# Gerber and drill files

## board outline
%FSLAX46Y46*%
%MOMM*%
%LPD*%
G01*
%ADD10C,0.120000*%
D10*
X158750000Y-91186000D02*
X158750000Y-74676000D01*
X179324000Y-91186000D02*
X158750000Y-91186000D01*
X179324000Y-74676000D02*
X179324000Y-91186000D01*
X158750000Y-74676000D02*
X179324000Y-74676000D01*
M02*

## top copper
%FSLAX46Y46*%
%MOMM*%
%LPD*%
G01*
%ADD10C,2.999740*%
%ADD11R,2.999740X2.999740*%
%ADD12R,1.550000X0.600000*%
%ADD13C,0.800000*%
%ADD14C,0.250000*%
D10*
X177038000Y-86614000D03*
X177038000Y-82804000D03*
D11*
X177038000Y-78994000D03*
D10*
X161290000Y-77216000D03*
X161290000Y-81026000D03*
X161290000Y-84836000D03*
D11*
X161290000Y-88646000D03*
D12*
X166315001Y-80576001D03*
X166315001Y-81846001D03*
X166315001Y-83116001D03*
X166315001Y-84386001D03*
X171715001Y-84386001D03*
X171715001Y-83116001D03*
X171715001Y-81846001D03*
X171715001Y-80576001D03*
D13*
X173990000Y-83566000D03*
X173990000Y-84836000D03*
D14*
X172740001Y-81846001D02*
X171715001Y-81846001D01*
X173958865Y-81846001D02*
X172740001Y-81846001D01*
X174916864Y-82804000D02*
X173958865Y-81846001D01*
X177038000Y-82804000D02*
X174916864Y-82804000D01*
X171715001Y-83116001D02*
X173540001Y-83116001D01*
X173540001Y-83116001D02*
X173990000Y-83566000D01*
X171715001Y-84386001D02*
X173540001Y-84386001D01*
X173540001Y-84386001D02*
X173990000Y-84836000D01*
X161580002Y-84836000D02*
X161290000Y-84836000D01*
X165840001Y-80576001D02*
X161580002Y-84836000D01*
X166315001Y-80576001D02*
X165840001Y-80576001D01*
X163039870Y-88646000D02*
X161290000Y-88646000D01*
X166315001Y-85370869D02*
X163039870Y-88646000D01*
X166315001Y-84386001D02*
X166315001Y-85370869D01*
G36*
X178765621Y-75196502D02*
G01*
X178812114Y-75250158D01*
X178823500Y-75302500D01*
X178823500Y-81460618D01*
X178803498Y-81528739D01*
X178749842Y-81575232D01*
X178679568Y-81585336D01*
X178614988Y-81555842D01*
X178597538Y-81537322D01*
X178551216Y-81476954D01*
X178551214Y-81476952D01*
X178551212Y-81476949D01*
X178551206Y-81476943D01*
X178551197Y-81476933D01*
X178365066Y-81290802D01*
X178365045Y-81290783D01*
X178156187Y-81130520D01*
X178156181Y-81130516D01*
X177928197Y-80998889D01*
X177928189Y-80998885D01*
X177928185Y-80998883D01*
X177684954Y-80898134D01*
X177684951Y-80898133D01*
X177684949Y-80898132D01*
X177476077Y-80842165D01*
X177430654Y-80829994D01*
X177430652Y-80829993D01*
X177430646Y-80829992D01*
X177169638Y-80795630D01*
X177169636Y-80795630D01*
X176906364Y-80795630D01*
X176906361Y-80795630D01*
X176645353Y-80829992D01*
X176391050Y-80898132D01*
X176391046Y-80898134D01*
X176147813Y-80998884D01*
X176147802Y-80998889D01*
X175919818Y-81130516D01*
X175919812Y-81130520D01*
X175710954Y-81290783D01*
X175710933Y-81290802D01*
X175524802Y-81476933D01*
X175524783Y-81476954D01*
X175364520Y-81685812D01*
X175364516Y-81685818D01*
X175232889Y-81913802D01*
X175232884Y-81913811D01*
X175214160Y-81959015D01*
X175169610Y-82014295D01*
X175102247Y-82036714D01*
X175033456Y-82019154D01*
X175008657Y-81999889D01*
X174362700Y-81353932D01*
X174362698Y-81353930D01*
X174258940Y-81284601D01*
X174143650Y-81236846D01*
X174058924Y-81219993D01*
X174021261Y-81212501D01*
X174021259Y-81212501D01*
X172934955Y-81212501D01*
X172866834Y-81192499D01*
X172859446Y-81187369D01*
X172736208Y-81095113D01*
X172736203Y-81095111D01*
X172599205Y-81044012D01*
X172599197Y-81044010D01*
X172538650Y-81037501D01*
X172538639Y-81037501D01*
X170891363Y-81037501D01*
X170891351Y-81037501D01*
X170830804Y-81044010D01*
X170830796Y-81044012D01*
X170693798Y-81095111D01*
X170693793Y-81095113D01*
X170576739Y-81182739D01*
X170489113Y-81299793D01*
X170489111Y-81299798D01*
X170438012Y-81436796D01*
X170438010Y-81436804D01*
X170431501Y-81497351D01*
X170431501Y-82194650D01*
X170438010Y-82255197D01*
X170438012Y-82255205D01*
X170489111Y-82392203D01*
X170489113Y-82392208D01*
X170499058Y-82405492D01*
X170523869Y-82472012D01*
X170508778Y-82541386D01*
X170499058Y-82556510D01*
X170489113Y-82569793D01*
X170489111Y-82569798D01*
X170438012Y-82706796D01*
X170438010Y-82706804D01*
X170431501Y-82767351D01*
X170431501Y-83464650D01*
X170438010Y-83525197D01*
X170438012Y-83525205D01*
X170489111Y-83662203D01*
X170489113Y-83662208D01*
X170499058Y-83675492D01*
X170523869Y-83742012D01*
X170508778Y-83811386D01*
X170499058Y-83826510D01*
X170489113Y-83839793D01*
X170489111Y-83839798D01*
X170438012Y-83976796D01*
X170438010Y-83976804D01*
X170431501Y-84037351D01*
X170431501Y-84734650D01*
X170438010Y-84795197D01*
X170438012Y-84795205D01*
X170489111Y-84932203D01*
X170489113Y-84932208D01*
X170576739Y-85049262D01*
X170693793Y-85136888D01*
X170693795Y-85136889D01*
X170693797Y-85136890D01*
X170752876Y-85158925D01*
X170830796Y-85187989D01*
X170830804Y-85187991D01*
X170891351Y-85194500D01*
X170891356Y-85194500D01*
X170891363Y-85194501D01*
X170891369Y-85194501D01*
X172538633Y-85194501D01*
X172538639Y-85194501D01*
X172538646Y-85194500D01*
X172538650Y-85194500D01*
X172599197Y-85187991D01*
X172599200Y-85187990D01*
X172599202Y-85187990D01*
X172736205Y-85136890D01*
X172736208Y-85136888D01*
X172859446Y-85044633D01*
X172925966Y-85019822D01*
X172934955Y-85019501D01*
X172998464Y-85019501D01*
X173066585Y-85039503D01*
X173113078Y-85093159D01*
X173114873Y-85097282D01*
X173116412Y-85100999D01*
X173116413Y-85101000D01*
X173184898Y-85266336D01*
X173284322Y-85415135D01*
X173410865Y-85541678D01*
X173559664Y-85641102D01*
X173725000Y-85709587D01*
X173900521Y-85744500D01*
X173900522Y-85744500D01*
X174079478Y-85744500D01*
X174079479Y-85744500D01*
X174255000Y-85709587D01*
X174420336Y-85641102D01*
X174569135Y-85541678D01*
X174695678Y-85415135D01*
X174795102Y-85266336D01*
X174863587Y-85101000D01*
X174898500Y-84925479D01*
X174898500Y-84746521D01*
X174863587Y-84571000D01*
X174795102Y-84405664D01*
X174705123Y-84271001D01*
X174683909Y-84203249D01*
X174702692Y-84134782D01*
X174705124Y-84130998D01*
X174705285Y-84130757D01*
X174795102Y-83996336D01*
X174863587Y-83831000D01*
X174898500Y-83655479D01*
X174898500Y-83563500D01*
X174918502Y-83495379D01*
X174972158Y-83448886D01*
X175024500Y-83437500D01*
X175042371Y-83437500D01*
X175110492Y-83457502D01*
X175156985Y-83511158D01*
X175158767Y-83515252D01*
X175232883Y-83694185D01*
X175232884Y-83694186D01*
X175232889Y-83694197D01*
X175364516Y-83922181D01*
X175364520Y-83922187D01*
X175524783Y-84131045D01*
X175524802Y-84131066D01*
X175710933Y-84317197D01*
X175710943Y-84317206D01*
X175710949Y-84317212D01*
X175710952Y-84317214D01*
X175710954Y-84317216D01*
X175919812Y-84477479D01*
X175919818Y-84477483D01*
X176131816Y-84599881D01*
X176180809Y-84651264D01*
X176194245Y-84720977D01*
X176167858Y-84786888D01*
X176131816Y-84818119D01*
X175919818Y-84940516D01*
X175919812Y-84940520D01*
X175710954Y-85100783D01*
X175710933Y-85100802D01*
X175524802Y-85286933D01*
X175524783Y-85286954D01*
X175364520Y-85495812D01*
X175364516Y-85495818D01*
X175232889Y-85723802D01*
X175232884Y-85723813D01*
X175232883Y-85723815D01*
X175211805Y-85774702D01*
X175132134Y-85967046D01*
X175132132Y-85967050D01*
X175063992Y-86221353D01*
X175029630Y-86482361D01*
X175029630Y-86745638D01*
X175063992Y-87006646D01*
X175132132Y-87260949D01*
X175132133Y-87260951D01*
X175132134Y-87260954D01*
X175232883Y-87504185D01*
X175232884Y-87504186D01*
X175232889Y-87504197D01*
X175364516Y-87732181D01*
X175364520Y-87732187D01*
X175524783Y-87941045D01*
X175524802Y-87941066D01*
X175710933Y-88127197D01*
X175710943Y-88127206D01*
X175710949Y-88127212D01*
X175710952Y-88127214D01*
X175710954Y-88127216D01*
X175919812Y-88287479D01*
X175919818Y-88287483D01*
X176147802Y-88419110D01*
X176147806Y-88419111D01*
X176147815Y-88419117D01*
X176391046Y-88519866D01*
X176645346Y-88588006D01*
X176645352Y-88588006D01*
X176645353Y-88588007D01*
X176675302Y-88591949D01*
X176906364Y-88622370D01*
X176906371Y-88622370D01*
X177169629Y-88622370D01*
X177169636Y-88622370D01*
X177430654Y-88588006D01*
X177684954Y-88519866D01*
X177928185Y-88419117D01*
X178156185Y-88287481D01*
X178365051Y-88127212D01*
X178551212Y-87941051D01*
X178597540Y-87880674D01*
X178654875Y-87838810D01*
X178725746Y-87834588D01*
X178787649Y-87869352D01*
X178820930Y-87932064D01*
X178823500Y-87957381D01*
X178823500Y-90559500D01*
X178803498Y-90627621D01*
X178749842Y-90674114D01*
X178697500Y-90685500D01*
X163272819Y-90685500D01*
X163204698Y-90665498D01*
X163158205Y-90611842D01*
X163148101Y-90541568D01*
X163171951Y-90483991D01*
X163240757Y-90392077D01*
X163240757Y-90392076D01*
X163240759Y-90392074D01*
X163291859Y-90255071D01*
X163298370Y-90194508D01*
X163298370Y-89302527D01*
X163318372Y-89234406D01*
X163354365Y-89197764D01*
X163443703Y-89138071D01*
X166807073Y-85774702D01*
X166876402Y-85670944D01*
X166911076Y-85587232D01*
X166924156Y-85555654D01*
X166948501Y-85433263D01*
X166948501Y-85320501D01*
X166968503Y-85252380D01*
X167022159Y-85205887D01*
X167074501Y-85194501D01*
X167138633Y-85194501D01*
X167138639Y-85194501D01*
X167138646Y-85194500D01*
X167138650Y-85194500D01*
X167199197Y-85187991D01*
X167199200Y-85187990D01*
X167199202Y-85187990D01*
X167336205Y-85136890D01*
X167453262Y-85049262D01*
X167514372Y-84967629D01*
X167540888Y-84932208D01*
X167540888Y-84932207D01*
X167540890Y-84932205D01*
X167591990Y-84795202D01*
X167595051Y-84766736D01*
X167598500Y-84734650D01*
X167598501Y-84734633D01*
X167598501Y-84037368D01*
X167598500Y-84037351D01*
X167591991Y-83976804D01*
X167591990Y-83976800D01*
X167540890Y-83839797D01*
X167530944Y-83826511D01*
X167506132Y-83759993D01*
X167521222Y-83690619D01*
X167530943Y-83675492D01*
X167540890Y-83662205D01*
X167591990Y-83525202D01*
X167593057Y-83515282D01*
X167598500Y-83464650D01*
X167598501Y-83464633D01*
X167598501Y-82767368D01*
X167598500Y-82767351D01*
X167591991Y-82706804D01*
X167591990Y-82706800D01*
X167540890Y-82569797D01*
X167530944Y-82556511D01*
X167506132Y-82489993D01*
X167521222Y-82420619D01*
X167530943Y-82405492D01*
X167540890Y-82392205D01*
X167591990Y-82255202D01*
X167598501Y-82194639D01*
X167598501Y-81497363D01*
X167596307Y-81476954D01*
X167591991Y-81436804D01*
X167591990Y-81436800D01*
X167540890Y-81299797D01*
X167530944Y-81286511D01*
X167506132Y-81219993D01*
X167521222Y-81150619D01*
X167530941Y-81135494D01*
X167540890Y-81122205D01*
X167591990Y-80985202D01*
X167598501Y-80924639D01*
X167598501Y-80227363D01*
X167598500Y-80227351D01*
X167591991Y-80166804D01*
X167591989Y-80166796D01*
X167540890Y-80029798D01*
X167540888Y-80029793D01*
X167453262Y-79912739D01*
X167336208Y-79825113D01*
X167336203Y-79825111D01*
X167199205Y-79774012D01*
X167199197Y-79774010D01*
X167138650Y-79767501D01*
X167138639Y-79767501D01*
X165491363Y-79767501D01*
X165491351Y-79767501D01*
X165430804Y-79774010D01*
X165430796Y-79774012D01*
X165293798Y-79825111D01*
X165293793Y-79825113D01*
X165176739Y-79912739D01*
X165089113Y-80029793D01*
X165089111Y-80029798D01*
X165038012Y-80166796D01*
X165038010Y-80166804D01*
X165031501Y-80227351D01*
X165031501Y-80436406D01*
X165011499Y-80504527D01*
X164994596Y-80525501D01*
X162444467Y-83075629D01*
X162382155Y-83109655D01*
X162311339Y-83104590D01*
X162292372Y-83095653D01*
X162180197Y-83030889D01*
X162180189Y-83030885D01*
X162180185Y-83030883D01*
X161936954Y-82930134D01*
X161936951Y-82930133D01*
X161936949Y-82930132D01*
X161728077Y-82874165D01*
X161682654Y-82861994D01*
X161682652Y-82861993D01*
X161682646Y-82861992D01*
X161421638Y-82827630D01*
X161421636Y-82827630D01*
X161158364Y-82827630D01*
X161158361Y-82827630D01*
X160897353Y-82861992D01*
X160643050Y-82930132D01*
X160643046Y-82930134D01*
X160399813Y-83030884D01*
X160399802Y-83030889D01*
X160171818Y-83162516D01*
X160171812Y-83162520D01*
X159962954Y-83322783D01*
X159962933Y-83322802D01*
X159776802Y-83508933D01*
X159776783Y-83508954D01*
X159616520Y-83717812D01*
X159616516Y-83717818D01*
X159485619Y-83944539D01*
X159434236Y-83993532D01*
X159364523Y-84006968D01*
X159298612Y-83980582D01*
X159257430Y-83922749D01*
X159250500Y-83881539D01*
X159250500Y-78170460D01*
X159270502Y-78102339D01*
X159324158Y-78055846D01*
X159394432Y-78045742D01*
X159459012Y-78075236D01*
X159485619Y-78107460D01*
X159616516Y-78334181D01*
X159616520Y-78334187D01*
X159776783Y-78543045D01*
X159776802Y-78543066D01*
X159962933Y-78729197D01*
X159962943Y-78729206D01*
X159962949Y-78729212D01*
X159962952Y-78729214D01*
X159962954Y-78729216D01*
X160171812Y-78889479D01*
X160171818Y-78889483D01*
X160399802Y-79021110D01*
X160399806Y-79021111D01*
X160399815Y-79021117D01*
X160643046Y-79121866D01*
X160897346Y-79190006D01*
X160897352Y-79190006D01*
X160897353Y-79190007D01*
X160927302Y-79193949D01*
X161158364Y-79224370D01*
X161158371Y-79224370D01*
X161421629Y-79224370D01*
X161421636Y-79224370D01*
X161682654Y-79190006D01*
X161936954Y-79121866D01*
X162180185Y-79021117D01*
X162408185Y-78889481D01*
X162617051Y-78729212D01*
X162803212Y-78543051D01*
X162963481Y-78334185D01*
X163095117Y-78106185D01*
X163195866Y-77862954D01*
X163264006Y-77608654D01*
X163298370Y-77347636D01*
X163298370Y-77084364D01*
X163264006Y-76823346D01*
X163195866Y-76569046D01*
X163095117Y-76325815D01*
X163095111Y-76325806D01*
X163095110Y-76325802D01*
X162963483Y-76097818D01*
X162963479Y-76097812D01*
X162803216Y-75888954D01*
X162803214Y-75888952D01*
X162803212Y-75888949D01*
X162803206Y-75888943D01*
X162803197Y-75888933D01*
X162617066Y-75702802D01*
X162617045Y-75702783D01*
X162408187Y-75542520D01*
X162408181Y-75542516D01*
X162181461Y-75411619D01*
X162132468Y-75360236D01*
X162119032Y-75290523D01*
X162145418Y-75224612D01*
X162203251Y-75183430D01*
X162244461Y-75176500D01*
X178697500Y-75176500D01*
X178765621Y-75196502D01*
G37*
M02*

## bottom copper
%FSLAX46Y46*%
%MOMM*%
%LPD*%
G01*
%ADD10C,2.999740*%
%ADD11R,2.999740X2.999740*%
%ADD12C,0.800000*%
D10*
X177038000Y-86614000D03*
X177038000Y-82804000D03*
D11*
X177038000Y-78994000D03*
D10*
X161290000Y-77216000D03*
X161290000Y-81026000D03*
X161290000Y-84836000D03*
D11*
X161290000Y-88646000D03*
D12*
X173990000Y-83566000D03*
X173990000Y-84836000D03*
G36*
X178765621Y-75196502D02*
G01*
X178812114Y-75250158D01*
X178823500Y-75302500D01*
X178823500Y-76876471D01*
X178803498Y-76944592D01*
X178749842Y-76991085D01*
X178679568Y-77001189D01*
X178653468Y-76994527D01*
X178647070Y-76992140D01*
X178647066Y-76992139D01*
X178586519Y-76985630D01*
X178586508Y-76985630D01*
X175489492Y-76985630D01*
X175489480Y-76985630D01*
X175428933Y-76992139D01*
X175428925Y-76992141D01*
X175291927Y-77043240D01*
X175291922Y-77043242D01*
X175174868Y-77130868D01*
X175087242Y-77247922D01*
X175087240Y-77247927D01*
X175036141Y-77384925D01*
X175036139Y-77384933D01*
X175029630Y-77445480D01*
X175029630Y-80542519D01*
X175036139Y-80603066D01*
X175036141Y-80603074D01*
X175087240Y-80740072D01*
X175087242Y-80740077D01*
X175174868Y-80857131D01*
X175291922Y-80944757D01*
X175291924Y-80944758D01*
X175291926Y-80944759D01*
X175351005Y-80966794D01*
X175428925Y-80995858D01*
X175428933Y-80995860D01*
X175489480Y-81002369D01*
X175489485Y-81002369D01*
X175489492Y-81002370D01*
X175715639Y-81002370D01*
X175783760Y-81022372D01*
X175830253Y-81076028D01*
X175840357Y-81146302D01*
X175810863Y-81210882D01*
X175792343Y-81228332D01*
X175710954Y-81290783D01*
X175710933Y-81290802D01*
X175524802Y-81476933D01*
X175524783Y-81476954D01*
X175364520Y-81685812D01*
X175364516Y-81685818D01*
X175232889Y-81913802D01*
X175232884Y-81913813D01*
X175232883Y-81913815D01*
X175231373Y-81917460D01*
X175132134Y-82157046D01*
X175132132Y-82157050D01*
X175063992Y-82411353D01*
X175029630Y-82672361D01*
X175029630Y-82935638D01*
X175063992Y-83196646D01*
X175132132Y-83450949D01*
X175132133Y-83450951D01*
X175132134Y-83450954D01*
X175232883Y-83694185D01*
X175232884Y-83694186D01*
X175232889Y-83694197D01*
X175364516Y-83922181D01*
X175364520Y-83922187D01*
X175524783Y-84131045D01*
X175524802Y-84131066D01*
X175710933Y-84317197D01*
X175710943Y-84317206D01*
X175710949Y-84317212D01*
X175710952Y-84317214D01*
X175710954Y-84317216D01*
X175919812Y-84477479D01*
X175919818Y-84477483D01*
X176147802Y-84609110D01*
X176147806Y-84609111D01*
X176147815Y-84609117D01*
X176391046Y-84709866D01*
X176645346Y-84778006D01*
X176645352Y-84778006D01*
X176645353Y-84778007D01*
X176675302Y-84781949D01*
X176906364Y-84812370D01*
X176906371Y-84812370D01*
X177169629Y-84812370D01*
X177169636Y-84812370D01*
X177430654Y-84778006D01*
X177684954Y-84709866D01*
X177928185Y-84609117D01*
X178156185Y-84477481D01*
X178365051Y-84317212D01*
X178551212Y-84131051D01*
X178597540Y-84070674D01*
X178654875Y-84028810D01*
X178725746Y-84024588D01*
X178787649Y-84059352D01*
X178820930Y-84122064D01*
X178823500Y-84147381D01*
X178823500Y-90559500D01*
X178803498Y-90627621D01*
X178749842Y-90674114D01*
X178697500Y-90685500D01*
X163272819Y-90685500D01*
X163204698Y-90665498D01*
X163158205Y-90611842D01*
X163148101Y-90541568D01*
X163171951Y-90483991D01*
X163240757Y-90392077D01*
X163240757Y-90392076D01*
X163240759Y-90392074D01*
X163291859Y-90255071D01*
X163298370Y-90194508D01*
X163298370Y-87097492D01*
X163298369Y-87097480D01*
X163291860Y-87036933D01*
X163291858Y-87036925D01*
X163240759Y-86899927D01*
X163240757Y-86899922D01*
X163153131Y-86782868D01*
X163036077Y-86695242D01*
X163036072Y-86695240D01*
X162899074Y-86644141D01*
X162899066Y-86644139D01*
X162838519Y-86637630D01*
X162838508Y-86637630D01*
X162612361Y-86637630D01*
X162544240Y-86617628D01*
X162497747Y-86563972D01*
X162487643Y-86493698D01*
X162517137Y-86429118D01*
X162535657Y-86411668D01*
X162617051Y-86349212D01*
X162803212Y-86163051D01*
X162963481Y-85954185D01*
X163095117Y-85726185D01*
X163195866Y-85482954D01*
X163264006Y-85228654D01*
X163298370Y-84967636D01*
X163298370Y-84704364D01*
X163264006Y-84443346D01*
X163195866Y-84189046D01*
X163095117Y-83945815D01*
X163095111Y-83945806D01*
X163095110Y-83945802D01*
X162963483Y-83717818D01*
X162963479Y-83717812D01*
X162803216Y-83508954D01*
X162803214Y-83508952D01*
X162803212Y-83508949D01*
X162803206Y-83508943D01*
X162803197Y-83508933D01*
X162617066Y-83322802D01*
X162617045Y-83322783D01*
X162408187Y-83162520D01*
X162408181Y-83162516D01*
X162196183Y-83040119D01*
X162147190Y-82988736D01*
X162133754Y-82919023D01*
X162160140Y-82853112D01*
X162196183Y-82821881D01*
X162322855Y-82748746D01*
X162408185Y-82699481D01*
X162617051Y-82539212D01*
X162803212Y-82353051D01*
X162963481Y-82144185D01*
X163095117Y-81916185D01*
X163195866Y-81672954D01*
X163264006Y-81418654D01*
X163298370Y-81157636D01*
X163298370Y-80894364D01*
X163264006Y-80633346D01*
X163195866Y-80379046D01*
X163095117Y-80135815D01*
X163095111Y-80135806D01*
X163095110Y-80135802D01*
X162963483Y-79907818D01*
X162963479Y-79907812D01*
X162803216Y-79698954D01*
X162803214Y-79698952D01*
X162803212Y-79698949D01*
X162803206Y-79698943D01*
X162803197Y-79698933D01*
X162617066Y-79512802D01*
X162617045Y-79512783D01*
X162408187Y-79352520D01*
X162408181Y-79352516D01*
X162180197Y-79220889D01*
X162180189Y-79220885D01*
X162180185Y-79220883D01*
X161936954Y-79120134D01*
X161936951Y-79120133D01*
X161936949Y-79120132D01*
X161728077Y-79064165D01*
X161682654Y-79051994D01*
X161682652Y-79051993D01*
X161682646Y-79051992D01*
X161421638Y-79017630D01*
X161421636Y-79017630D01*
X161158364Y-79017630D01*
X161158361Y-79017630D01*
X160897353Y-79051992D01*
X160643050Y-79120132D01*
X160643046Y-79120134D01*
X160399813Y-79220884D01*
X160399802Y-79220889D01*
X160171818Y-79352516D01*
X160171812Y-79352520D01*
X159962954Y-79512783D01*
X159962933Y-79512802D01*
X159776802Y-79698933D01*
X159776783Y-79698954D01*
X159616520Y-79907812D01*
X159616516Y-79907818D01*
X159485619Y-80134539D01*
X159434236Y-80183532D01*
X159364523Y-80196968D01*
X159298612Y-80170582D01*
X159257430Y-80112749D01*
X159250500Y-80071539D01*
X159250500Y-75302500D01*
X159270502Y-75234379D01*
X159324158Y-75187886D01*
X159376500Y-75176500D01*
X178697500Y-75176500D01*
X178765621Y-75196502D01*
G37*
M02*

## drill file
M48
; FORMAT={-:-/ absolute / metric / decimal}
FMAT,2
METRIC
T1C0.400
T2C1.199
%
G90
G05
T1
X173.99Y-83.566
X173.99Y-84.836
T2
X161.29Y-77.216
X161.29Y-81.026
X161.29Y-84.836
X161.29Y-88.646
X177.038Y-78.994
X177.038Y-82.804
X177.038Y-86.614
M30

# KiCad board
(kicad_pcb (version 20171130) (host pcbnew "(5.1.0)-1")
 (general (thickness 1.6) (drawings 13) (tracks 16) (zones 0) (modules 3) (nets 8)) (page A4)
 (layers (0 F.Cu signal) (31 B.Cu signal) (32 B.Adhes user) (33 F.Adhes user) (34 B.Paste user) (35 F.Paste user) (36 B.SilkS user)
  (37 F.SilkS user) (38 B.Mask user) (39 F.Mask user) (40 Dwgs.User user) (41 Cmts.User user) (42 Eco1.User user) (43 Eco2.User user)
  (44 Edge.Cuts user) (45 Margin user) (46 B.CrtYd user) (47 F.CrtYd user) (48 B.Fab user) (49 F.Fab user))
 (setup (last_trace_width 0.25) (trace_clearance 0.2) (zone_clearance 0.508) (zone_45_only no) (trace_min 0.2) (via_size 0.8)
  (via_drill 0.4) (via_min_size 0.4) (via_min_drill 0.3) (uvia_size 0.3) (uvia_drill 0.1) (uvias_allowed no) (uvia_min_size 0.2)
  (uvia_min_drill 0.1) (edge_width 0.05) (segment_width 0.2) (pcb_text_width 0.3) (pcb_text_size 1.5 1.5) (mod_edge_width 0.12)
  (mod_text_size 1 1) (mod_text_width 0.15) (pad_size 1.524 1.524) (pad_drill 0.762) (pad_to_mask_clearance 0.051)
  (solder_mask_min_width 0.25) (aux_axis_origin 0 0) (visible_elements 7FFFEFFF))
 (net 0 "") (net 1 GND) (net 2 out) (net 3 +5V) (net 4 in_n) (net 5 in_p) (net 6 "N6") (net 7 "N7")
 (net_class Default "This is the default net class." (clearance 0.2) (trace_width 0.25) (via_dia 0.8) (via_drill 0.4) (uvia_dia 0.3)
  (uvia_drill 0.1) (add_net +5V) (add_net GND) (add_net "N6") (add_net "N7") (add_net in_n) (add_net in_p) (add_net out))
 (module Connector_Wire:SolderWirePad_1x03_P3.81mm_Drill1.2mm (layer F.Cu) (at 177.038 78.994 270)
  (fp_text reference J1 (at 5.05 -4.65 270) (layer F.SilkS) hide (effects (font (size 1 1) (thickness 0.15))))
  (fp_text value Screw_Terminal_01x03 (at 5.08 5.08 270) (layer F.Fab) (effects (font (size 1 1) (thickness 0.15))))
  (pad 3 thru_hole circle (at 7.62 0 270) (size 2.99974 2.99974) (drill 1.19888) (layers *.Cu *.Mask) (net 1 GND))
  (pad 2 thru_hole circle (at 3.81 0 270) (size 2.99974 2.99974) (drill 1.19888) (layers *.Cu *.Mask) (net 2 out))
  (pad 1 thru_hole rect (at 0 0 270) (size 2.99974 2.99974) (drill 1.19888) (layers *.Cu *.Mask) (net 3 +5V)))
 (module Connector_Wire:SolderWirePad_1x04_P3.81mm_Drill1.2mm (layer F.Cu) (at 161.29 88.646 90)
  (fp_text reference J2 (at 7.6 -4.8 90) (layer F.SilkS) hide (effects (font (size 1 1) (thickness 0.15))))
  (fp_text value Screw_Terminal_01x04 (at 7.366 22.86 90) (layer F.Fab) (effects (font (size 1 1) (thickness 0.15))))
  (pad 4 thru_hole circle (at 11.43 0 90) (size 2.99974 2.99974) (drill 1.19888) (layers *.Cu *.Mask) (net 1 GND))
  (pad 3 thru_hole circle (at 7.62 0 90) (size 2.99974 2.99974) (drill 1.19888) (layers *.Cu *.Mask) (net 3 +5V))
  (pad 2 thru_hole circle (at 3.81 0 90) (size 2.99974 2.99974) (drill 1.19888) (layers *.Cu *.Mask) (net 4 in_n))
  (pad 1 thru_hole rect (at 0 0 90) (size 2.99974 2.99974) (drill 1.19888) (layers *.Cu *.Mask) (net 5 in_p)))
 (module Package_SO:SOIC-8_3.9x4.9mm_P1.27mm (layer F.Cu) (at 169.015001 82.481001)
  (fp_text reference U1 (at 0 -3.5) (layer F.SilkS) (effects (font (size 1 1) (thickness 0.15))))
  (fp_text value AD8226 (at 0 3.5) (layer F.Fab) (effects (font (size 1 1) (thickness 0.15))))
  (pad 1 smd rect (at -2.7 -1.905) (size 1.55 0.6) (layers F.Cu F.Paste F.Mask) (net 4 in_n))
  (pad 2 smd rect (at -2.7 -0.635) (size 1.55 0.6) (layers F.Cu F.Paste F.Mask) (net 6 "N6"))
  (pad 3 smd rect (at -2.7 0.635) (size 1.55 0.6) (layers F.Cu F.Paste F.Mask) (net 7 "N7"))
  (pad 4 smd rect (at -2.7 1.905) (size 1.55 0.6) (layers F.Cu F.Paste F.Mask) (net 5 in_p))
  (pad 5 smd rect (at 2.7 1.905) (size 1.55 0.6) (layers F.Cu F.Paste F.Mask) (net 1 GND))
  (pad 6 smd rect (at 2.7 0.635) (size 1.55 0.6) (layers F.Cu F.Paste F.Mask) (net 1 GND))
  (pad 7 smd rect (at 2.7 -0.635) (size 1.55 0.6) (layers F.Cu F.Paste F.Mask) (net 2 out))
  (pad 8 smd rect (at 2.7 -1.905) (size 1.55 0.6) (layers F.Cu F.Paste F.Mask) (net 3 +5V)))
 (gr_line (start 158.75 91.186) (end 158.75 74.676) (layer Edge.Cuts) (width 0.12))
 (gr_line (start 179.324 91.186) (end 158.75 91.186) (layer Edge.Cuts) (width 0.12))
 (gr_line (start 179.324 74.676) (end 179.324 91.186) (layer Edge.Cuts) (width 0.12))
 (gr_line (start 158.75 74.676) (end 179.324 74.676) (layer Edge.Cuts) (width 0.12))
 (segment (start 172.740001 81.846001) (end 171.715001 81.846001) (width 0.25) (layer F.Cu) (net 2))
 (segment (start 173.958865 81.846001) (end 172.740001 81.846001) (width 0.25) (layer F.Cu) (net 2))
 (segment (start 174.916864 82.804) (end 173.958865 81.846001) (width 0.25) (layer F.Cu) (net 2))
 (segment (start 177.038 82.804) (end 174.916864 82.804) (width 0.25) (layer F.Cu) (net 2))
 (via (at 173.99 83.566) (size 0.8) (drill 0.4) (layers F.Cu B.Cu) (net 1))
 (segment (start 171.715001 83.116001) (end 173.540001 83.116001) (width 0.25) (layer F.Cu) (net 1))
 (segment (start 173.540001 83.116001) (end 173.99 83.566) (width 0.25) (layer F.Cu) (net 1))
 (via (at 173.99 84.836) (size 0.8) (drill 0.4) (layers F.Cu B.Cu) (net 1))
 (segment (start 171.715001 84.386001) (end 173.540001 84.386001) (width 0.25) (layer F.Cu) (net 1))
 (segment (start 173.540001 84.386001) (end 173.99 84.836) (width 0.25) (layer F.Cu) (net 1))
 (segment (start 161.580002 84.836) (end 161.29 84.836) (width 0.25) (layer F.Cu) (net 4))
 (segment (start 165.840001 80.576001) (end 161.580002 84.836) (width 0.25) (layer F.Cu) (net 4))
 (segment (start 166.315001 80.576001) (end 165.840001 80.576001) (width 0.25) (layer F.Cu) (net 4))
 (segment (start 163.03987 88.646) (end 161.29 88.646) (width 0.25) (layer F.Cu) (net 5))
 (segment (start 166.315001 85.370869) (end 163.03987 88.646) (width 0.25) (layer F.Cu) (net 5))
 (segment (start 166.315001 84.386001) (end 166.315001 85.370869) (width 0.25) (layer F.Cu) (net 5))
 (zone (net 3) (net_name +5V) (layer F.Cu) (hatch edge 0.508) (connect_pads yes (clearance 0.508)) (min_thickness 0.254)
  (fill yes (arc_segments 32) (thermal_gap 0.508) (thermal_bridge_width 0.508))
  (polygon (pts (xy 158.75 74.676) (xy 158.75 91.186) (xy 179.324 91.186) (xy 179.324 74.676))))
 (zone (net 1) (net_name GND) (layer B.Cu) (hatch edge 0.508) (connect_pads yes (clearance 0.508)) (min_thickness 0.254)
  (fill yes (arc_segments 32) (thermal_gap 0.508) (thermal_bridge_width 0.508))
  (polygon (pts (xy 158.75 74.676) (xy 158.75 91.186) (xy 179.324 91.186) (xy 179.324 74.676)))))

